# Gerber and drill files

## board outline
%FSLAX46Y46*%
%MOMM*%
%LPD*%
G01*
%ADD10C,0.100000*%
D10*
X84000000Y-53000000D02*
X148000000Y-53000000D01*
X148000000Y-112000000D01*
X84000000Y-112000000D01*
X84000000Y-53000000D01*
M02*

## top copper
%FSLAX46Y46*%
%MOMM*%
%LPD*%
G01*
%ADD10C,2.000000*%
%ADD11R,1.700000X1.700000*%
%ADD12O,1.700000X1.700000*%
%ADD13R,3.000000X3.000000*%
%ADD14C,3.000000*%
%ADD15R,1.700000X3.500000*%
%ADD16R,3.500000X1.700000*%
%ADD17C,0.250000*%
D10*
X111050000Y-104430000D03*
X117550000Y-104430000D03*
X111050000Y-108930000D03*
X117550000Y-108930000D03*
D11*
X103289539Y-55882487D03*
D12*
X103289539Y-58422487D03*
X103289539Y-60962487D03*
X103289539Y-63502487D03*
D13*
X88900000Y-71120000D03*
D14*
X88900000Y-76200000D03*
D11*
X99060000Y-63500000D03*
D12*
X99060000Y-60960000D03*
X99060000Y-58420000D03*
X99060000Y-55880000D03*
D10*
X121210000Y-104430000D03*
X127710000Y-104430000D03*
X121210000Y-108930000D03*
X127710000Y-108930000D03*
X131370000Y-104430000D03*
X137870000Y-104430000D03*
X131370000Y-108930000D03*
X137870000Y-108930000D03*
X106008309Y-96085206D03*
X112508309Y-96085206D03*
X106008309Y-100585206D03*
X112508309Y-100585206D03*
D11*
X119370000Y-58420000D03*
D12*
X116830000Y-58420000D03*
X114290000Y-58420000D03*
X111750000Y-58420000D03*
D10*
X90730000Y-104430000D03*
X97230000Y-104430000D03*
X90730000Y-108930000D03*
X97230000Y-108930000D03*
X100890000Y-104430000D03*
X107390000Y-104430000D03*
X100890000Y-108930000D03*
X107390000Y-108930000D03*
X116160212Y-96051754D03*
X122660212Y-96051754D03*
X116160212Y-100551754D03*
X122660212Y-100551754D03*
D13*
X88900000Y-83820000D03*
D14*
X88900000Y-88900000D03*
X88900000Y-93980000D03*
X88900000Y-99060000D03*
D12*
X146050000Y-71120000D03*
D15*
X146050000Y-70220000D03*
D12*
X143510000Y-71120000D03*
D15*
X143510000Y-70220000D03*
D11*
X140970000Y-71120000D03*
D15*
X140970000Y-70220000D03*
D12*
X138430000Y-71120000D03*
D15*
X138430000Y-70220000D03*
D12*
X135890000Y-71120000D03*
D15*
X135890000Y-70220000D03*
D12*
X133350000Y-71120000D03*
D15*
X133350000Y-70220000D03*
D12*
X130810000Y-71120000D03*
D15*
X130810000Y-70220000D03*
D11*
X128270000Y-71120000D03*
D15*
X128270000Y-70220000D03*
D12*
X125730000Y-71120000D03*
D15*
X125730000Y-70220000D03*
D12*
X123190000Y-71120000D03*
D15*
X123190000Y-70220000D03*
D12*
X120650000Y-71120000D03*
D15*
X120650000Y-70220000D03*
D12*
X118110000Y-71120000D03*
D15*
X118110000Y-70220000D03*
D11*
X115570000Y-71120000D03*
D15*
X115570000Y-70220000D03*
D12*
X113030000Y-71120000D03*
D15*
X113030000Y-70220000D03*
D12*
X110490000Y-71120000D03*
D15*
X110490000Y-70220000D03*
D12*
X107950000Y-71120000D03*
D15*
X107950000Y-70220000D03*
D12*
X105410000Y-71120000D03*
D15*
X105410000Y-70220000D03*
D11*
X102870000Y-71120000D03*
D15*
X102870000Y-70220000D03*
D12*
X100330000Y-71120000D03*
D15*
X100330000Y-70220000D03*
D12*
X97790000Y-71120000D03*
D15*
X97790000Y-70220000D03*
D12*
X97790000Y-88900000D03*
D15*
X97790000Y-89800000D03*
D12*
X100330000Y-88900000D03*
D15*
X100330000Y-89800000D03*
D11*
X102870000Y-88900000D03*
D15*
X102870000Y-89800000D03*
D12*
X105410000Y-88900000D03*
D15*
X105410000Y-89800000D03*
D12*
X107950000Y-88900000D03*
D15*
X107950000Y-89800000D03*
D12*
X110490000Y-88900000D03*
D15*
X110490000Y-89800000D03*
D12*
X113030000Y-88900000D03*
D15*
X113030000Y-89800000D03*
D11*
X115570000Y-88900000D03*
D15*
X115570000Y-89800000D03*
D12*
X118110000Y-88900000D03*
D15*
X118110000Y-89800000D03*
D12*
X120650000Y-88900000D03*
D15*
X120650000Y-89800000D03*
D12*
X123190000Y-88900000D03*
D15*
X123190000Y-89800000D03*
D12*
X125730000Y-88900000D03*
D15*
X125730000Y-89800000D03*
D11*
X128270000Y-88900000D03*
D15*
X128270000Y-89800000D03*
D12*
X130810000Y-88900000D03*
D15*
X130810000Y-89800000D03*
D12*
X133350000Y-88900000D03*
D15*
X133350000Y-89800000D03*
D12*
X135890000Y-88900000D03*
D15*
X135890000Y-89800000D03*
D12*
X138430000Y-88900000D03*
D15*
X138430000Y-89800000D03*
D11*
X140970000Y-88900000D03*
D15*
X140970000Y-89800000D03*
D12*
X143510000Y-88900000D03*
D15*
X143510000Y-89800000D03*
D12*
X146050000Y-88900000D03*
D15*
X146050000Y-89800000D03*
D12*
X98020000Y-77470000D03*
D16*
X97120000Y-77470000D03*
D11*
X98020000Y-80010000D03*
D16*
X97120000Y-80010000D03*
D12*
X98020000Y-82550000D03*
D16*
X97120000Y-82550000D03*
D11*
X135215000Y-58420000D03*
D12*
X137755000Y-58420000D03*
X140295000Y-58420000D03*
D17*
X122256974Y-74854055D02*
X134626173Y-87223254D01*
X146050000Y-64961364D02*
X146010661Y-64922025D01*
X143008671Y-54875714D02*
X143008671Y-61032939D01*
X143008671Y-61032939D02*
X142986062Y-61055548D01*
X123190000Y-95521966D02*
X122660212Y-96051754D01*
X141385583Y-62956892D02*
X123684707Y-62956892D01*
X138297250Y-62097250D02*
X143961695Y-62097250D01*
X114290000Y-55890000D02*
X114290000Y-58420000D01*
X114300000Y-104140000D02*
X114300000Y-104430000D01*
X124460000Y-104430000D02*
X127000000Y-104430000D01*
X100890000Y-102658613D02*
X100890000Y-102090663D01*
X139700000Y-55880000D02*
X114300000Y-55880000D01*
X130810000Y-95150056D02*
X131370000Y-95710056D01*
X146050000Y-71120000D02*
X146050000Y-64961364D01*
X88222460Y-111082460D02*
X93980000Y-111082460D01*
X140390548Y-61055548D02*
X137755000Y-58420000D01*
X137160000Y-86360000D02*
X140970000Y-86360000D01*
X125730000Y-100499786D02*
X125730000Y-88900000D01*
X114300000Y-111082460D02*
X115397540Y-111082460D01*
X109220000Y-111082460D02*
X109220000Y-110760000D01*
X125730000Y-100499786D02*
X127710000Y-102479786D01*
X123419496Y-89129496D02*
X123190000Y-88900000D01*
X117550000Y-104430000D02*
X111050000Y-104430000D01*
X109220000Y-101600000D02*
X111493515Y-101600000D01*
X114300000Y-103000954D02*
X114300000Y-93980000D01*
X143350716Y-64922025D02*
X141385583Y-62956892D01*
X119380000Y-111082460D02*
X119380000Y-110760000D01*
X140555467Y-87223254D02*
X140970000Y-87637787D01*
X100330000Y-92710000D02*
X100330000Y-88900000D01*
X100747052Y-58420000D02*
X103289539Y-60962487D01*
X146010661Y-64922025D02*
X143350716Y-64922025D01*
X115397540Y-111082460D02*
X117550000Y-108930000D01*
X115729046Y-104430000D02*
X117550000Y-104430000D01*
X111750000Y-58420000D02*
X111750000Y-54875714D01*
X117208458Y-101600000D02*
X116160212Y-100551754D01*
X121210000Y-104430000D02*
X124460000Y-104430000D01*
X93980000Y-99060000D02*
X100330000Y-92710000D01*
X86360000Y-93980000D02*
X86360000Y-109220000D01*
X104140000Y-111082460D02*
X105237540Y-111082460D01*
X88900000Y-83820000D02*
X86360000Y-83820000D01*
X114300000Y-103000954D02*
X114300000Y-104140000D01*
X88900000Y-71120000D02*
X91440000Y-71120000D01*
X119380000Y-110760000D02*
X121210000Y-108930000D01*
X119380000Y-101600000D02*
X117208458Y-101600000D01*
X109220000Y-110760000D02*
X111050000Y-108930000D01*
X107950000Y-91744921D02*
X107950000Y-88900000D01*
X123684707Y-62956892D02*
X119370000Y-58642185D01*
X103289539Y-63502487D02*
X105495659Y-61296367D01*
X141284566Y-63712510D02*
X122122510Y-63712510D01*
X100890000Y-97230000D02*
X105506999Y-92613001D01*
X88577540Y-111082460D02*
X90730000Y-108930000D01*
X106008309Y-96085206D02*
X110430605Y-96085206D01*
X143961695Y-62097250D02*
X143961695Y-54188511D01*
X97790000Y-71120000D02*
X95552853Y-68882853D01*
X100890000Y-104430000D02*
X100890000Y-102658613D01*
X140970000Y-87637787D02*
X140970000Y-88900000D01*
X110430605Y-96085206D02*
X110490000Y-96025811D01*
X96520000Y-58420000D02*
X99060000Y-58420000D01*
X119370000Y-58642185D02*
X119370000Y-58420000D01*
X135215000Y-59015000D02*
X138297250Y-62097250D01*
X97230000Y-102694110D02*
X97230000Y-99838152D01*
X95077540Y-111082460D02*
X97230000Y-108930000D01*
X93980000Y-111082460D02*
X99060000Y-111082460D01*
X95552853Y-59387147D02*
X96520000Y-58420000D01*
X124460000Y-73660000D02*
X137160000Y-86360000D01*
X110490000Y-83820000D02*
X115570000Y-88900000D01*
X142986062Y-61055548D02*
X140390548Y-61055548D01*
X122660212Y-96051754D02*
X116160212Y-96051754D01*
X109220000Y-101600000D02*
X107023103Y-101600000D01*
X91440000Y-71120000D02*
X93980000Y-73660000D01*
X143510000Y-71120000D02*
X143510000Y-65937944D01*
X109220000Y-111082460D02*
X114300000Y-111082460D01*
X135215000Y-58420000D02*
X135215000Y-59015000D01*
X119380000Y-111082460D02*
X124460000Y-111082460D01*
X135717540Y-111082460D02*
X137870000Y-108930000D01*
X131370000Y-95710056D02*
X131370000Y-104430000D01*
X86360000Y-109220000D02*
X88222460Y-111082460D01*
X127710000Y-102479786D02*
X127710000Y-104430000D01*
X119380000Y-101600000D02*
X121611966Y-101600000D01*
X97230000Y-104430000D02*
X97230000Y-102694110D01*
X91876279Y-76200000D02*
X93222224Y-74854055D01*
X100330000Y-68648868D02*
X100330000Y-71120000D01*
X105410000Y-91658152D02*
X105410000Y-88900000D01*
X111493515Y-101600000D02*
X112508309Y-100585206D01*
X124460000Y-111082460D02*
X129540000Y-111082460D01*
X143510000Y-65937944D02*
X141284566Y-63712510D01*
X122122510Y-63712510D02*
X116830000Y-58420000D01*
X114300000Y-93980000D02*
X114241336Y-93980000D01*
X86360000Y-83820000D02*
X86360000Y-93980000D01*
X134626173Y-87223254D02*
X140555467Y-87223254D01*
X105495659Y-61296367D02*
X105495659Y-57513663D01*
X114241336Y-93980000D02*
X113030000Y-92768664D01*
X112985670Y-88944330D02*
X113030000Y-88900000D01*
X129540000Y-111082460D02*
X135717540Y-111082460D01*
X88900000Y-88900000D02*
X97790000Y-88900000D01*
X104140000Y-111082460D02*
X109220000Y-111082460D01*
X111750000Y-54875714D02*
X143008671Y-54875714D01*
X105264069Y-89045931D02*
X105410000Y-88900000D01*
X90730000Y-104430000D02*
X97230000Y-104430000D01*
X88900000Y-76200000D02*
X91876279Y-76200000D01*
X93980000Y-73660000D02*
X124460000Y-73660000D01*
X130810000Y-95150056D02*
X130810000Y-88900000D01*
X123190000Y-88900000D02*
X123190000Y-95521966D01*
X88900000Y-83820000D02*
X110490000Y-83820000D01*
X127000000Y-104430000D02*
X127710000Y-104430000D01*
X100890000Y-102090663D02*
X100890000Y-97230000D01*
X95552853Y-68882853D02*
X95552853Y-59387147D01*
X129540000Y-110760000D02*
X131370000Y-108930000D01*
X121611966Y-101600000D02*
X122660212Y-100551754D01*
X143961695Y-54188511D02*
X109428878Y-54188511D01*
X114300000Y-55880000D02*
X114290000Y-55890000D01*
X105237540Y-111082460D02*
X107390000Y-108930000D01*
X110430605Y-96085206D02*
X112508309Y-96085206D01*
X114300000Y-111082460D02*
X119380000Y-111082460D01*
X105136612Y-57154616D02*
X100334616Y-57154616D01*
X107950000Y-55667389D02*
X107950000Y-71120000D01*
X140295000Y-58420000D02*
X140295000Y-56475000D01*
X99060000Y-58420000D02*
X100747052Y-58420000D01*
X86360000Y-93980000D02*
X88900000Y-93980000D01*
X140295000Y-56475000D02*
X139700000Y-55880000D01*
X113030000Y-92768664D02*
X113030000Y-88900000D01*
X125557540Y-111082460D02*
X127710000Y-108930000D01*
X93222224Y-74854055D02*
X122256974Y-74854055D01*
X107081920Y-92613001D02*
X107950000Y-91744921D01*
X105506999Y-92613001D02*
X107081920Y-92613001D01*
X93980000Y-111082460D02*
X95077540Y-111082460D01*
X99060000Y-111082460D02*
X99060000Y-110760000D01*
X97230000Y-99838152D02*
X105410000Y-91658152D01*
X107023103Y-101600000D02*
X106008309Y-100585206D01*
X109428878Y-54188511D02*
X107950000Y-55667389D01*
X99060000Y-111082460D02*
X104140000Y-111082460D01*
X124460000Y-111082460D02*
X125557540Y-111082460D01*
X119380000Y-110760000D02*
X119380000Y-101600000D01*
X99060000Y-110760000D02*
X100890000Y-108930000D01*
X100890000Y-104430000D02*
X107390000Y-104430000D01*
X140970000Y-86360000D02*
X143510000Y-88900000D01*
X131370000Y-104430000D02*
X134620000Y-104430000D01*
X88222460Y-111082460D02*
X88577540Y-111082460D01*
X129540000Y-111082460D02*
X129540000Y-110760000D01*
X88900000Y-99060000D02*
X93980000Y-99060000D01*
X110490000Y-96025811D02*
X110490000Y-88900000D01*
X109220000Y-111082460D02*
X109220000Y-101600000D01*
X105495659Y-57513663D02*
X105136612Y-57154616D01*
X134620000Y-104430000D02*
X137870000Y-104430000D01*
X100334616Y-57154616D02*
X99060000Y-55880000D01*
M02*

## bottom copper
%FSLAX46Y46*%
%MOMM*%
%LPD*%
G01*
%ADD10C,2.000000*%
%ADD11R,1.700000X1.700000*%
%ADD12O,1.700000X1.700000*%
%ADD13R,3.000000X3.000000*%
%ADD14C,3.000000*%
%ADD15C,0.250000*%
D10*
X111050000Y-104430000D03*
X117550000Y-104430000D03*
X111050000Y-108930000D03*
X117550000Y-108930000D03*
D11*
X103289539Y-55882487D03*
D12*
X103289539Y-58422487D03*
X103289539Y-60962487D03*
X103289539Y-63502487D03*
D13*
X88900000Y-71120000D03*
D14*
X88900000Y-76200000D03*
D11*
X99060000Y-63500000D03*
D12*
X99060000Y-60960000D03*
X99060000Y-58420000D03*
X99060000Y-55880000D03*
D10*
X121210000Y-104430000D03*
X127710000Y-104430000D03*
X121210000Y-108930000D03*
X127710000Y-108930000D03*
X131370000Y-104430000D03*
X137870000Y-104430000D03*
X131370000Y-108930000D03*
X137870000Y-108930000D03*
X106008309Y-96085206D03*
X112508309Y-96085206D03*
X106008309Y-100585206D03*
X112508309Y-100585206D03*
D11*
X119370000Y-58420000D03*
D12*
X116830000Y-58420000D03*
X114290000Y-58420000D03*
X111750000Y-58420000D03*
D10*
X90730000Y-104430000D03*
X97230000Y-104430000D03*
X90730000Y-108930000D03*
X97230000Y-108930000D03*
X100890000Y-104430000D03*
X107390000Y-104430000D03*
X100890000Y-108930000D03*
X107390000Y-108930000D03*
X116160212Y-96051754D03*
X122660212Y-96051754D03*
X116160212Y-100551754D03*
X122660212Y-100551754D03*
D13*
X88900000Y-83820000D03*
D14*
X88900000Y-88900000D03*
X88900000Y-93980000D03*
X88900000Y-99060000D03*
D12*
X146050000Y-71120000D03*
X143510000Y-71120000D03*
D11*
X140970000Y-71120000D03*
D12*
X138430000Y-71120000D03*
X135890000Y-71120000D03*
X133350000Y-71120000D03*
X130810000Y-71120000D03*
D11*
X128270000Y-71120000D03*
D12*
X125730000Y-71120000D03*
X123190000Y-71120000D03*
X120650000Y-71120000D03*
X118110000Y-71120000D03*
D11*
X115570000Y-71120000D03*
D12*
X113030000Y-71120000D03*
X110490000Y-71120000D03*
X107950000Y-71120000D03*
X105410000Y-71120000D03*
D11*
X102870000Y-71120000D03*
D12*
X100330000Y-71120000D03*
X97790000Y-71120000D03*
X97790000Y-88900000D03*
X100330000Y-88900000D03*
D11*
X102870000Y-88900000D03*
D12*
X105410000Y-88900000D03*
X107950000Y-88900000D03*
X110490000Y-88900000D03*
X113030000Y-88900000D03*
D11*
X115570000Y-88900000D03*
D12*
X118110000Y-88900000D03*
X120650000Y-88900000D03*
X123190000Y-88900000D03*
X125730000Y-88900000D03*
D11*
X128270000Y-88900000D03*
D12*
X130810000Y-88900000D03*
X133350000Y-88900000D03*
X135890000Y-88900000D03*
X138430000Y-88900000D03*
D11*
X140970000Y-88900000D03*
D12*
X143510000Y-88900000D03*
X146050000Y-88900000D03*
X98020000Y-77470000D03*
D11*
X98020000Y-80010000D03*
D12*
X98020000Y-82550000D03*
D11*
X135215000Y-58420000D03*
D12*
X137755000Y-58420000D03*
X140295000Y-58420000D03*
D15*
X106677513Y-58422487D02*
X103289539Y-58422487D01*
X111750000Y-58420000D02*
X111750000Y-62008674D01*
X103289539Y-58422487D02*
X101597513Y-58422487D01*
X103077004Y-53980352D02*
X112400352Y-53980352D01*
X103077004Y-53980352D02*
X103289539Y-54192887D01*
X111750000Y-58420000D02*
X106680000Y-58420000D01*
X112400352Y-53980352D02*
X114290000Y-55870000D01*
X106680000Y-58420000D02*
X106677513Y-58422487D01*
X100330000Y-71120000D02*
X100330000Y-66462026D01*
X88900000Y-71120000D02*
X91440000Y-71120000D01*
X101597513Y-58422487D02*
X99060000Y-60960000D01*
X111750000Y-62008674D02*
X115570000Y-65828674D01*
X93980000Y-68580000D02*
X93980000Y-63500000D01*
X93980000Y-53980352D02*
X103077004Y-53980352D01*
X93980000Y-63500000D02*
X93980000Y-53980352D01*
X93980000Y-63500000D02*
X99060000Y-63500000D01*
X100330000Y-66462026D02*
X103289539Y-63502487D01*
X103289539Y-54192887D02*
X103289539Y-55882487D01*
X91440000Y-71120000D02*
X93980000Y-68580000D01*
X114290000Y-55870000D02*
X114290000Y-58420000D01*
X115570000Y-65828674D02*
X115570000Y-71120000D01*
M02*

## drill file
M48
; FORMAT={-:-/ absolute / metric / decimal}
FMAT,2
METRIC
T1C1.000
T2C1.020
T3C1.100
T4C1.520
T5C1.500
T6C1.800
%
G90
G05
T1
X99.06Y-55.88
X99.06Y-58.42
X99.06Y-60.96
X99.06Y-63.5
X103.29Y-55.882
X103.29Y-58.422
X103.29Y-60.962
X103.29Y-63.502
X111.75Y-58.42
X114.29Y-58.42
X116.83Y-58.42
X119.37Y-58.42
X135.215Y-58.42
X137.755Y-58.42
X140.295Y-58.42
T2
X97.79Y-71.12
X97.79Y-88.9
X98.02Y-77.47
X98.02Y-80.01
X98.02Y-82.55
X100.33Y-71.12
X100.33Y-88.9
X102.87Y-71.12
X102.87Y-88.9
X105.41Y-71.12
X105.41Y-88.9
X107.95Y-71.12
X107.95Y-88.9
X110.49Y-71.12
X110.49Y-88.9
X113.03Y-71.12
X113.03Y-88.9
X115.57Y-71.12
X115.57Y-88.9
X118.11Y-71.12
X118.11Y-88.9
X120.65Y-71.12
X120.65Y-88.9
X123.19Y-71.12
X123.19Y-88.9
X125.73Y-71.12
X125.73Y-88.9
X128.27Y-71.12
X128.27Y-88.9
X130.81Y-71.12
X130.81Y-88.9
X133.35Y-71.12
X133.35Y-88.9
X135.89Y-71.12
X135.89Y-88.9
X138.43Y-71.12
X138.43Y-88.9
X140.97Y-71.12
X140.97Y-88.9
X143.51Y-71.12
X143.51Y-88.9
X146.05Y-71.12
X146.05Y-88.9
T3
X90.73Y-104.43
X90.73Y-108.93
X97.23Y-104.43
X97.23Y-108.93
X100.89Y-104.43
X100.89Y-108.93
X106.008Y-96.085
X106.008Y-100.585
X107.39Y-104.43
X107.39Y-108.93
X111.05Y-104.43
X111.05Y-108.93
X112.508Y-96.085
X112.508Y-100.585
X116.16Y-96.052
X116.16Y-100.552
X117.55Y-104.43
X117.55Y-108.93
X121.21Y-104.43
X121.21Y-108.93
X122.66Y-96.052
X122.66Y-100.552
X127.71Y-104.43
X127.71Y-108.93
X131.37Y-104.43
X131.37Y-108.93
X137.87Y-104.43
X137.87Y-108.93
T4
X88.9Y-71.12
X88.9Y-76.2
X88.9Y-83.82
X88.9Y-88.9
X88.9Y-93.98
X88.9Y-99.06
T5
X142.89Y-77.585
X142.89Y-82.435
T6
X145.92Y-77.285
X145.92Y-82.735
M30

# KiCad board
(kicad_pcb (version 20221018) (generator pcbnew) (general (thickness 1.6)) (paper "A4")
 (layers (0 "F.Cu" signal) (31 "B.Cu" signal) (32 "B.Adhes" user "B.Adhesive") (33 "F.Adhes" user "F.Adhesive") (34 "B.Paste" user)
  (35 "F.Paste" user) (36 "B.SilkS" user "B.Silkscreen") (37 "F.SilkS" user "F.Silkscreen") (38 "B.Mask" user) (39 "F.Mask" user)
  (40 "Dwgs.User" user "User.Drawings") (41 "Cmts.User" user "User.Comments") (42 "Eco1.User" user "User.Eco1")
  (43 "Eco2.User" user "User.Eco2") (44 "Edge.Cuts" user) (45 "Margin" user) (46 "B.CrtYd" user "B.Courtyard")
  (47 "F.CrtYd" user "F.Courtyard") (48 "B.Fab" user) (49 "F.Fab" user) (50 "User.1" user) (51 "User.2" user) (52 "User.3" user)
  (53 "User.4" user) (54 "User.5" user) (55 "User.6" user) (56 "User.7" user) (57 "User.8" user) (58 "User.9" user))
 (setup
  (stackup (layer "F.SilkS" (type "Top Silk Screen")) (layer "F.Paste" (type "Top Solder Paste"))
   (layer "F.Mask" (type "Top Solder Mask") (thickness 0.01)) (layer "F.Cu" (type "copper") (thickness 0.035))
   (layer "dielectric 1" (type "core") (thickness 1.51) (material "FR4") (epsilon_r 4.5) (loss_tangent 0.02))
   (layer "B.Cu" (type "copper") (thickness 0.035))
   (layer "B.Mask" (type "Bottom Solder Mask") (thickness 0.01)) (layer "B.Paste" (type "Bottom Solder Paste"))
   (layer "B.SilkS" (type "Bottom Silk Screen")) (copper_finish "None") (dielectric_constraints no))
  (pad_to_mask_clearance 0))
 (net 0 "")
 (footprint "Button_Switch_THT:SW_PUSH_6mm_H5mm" (layer "F.Cu") (at 111.05 104.43)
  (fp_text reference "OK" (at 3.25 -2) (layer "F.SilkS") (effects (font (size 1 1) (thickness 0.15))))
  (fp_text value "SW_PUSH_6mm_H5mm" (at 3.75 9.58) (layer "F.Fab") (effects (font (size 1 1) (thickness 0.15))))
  (pad "1" thru_hole circle (at 0 0 90) (size 2 2) (drill 1.1) (layers "*.Cu" "*.Mask"))
  (pad "1" thru_hole circle (at 6.5 0 90) (size 2 2) (drill 1.1) (layers "*.Cu" "*.Mask"))
  (pad "2" thru_hole circle (at 0 4.5 90) (size 2 2) (drill 1.1) (layers "*.Cu" "*.Mask"))
  (pad "2" thru_hole circle (at 6.5 4.5 90) (size 2 2) (drill 1.1) (layers "*.Cu" "*.Mask")))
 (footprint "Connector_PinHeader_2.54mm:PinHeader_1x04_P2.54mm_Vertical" (layer "F.Cu") (at 103.289539 55.882487)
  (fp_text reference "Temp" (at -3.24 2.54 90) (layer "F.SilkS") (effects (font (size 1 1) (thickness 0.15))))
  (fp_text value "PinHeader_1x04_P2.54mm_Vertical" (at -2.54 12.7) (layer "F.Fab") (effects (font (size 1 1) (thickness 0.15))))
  (pad "1" thru_hole rect (at 0 0) (size 1.7 1.7) (drill 1) (layers "*.Cu" "*.Mask"))
  (pad "2" thru_hole oval (at 0 2.54) (size 1.7 1.7) (drill 1) (layers "*.Cu" "*.Mask"))
  (pad "3" thru_hole oval (at 0 5.08) (size 1.7 1.7) (drill 1) (layers "*.Cu" "*.Mask"))
  (pad "4" thru_hole oval (at 0 7.62) (size 1.7 1.7) (drill 1) (layers "*.Cu" "*.Mask")))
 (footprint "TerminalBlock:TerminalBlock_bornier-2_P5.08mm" (layer "F.Cu") (at 88.9 71.12 -90)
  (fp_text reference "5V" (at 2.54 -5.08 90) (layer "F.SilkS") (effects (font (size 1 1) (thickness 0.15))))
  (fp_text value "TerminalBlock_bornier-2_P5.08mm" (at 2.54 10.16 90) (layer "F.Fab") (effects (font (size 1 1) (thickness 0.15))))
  (pad "1" thru_hole rect (at 0 0 270) (size 3 3) (drill 1.52) (layers "*.Cu" "*.Mask"))
  (pad "2" thru_hole circle (at 5.08 0 270) (size 3 3) (drill 1.52) (layers "*.Cu" "*.Mask")))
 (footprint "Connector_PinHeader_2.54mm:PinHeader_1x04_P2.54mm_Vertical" (layer "F.Cu") (at 99.06 63.5 180)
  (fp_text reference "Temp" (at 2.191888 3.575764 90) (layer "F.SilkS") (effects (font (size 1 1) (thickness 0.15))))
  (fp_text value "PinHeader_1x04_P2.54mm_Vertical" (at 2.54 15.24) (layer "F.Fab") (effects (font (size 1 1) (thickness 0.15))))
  (pad "1" thru_hole rect (at 0 0 180) (size 1.7 1.7) (drill 1) (layers "*.Cu" "*.Mask"))
  (pad "2" thru_hole oval (at 0 2.54 180) (size 1.7 1.7) (drill 1) (layers "*.Cu" "*.Mask"))
  (pad "3" thru_hole oval (at 0 5.08 180) (size 1.7 1.7) (drill 1) (layers "*.Cu" "*.Mask"))
  (pad "4" thru_hole oval (at 0 7.62 180) (size 1.7 1.7) (drill 1) (layers "*.Cu" "*.Mask")))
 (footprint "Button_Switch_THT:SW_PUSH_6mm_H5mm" (layer "F.Cu") (at 121.21 104.43)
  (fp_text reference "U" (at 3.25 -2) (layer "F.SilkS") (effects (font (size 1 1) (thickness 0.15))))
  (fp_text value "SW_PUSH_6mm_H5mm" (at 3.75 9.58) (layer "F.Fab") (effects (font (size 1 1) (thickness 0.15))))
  (pad "1" thru_hole circle (at 0 0 90) (size 2 2) (drill 1.1) (layers "*.Cu" "*.Mask"))
  (pad "1" thru_hole circle (at 6.5 0 90) (size 2 2) (drill 1.1) (layers "*.Cu" "*.Mask"))
  (pad "2" thru_hole circle (at 0 4.5 90) (size 2 2) (drill 1.1) (layers "*.Cu" "*.Mask"))
  (pad "2" thru_hole circle (at 6.5 4.5 90) (size 2 2) (drill 1.1) (layers "*.Cu" "*.Mask")))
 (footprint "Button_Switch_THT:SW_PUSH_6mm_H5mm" (layer "F.Cu") (at 131.37 104.43)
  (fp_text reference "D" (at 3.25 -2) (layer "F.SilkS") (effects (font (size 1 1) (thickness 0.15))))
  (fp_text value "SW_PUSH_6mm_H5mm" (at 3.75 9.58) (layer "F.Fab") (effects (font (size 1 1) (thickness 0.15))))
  (pad "1" thru_hole circle (at 0 0 90) (size 2 2) (drill 1.1) (layers "*.Cu" "*.Mask"))
  (pad "1" thru_hole circle (at 6.5 0 90) (size 2 2) (drill 1.1) (layers "*.Cu" "*.Mask"))
  (pad "2" thru_hole circle (at 0 4.5 90) (size 2 2) (drill 1.1) (layers "*.Cu" "*.Mask"))
  (pad "2" thru_hole circle (at 6.5 4.5 90) (size 2 2) (drill 1.1) (layers "*.Cu" "*.Mask")))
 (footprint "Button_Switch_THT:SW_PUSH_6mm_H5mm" (layer "F.Cu") (at 106.008309 96.085206)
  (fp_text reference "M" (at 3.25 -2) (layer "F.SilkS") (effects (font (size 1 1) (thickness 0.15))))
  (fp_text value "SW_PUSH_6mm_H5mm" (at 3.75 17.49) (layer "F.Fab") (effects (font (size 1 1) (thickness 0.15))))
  (pad "1" thru_hole circle (at 0 0 90) (size 2 2) (drill 1.1) (layers "*.Cu" "*.Mask"))
  (pad "1" thru_hole circle (at 6.5 0 90) (size 2 2) (drill 1.1) (layers "*.Cu" "*.Mask"))
  (pad "2" thru_hole circle (at 0 4.5 90) (size 2 2) (drill 1.1) (layers "*.Cu" "*.Mask"))
  (pad "2" thru_hole circle (at 6.5 4.5 90) (size 2 2) (drill 1.1) (layers "*.Cu" "*.Mask")))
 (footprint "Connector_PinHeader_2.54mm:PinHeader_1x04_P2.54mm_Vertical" (layer "F.Cu") (at 119.37 58.42 -90)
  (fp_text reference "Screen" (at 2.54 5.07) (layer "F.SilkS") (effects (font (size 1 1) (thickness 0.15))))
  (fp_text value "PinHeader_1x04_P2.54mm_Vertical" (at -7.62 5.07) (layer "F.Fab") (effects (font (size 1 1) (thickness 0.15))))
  (pad "1" thru_hole rect (at 0 0 270) (size 1.7 1.7) (drill 1) (layers "*.Cu" "*.Mask"))
  (pad "2" thru_hole oval (at 0 2.54 270) (size 1.7 1.7) (drill 1) (layers "*.Cu" "*.Mask"))
  (pad "3" thru_hole oval (at 0 5.08 270) (size 1.7 1.7) (drill 1) (layers "*.Cu" "*.Mask"))
  (pad "4" thru_hole oval (at 0 7.62 270) (size 1.7 1.7) (drill 1) (layers "*.Cu" "*.Mask")))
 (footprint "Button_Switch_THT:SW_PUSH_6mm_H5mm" (layer "F.Cu") (at 90.73 104.43)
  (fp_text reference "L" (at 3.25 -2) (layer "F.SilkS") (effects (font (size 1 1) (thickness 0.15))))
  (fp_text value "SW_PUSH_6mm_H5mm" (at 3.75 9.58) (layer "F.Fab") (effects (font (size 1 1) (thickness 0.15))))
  (pad "1" thru_hole circle (at 0 0 90) (size 2 2) (drill 1.1) (layers "*.Cu" "*.Mask"))
  (pad "1" thru_hole circle (at 6.5 0 90) (size 2 2) (drill 1.1) (layers "*.Cu" "*.Mask"))
  (pad "2" thru_hole circle (at 0 4.5 90) (size 2 2) (drill 1.1) (layers "*.Cu" "*.Mask"))
  (pad "2" thru_hole circle (at 6.5 4.5 90) (size 2 2) (drill 1.1) (layers "*.Cu" "*.Mask")))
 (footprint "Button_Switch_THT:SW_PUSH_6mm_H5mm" (layer "F.Cu") (at 100.89 104.43)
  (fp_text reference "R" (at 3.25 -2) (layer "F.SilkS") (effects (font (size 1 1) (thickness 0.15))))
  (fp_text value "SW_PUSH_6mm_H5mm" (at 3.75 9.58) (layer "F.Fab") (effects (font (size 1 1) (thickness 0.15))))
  (pad "1" thru_hole circle (at 0 0 90) (size 2 2) (drill 1.1) (layers "*.Cu" "*.Mask"))
  (pad "1" thru_hole circle (at 6.5 0 90) (size 2 2) (drill 1.1) (layers "*.Cu" "*.Mask"))
  (pad "2" thru_hole circle (at 0 4.5 90) (size 2 2) (drill 1.1) (layers "*.Cu" "*.Mask"))
  (pad "2" thru_hole circle (at 6.5 4.5 90) (size 2 2) (drill 1.1) (layers "*.Cu" "*.Mask")))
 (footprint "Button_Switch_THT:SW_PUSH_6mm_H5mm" (layer "F.Cu") (at 116.160212 96.051754)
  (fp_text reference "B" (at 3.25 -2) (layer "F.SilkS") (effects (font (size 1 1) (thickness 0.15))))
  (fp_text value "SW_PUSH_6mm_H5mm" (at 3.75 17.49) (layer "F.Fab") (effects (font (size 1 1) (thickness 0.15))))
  (pad "1" thru_hole circle (at 0 0 90) (size 2 2) (drill 1.1) (layers "*.Cu" "*.Mask"))
  (pad "1" thru_hole circle (at 6.5 0 90) (size 2 2) (drill 1.1) (layers "*.Cu" "*.Mask"))
  (pad "2" thru_hole circle (at 0 4.5 90) (size 2 2) (drill 1.1) (layers "*.Cu" "*.Mask"))
  (pad "2" thru_hole circle (at 6.5 4.5 90) (size 2 2) (drill 1.1) (layers "*.Cu" "*.Mask")))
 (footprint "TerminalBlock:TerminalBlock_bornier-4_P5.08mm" (layer "F.Cu") (at 88.9 83.82 -90)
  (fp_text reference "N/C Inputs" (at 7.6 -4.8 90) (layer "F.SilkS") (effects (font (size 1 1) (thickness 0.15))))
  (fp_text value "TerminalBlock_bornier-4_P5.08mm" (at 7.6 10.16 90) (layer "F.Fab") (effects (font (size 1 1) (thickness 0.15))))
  (pad "1" thru_hole rect (at 0 0 270) (size 3 3) (drill 1.52) (layers "*.Cu" "*.Mask"))
  (pad "2" thru_hole circle (at 5.08 0 270) (size 3 3) (drill 1.52) (layers "*.Cu" "*.Mask"))
  (pad "3" thru_hole circle (at 10.16 0 270) (size 3 3) (drill 1.52) (layers "*.Cu" "*.Mask"))
  (pad "4" thru_hole circle (at 15.24 0 270) (size 3 3) (drill 1.52) (layers "*.Cu" "*.Mask")))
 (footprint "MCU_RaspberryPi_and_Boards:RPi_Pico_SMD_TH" (layer "F.Cu") (at 121.92 80.01 -90)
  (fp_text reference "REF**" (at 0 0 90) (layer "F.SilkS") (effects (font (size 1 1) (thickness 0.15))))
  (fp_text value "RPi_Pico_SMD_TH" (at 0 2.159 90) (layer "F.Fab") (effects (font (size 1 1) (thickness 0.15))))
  (pad "" np_thru_hole oval (at -2.725 -24 270) (size 1.8 1.8) (drill 1.8) (layers "*.Cu" "*.Mask"))
  (pad "" np_thru_hole oval (at -2.425 -20.97 270) (size 1.5 1.5) (drill 1.5) (layers "*.Cu" "*.Mask"))
  (pad "" np_thru_hole oval (at 2.425 -20.97 270) (size 1.5 1.5) (drill 1.5) (layers "*.Cu" "*.Mask"))
  (pad "" np_thru_hole oval (at 2.725 -24 270) (size 1.8 1.8) (drill 1.8) (layers "*.Cu" "*.Mask"))
  (pad "1" thru_hole oval (at -8.89 -24.13 270) (size 1.7 1.7) (drill 1.02) (layers "*.Cu" "*.Mask"))
  (pad "1" smd rect (at -8.89 -24.13 270) (size 3.5 1.7) (drill (offset -0.9 0)) (layers "F.Cu" "F.Mask"))
  (pad "2" thru_hole oval (at -8.89 -21.59 270) (size 1.7 1.7) (drill 1.02) (layers "*.Cu" "*.Mask"))
  (pad "2" smd rect (at -8.89 -21.59 270) (size 3.5 1.7) (drill (offset -0.9 0)) (layers "F.Cu" "F.Mask"))
  (pad "3" thru_hole rect (at -8.89 -19.05 270) (size 1.7 1.7) (drill 1.02) (layers "*.Cu" "*.Mask"))
  (pad "3" smd rect (at -8.89 -19.05 270) (size 3.5 1.7) (drill (offset -0.9 0)) (layers "F.Cu" "F.Mask"))
  (pad "4" thru_hole oval (at -8.89 -16.51 270) (size 1.7 1.7) (drill 1.02) (layers "*.Cu" "*.Mask"))
  (pad "4" smd rect (at -8.89 -16.51 270) (size 3.5 1.7) (drill (offset -0.9 0)) (layers "F.Cu" "F.Mask"))
  (pad "5" thru_hole oval (at -8.89 -13.97 270) (size 1.7 1.7) (drill 1.02) (layers "*.Cu" "*.Mask"))
  (pad "5" smd rect (at -8.89 -13.97 270) (size 3.5 1.7) (drill (offset -0.9 0)) (layers "F.Cu" "F.Mask"))
  (pad "6" thru_hole oval (at -8.89 -11.43 270) (size 1.7 1.7) (drill 1.02) (layers "*.Cu" "*.Mask"))
  (pad "6" smd rect (at -8.89 -11.43 270) (size 3.5 1.7) (drill (offset -0.9 0)) (layers "F.Cu" "F.Mask"))
  (pad "7" thru_hole oval (at -8.89 -8.89 270) (size 1.7 1.7) (drill 1.02) (layers "*.Cu" "*.Mask"))
  (pad "7" smd rect (at -8.89 -8.89 270) (size 3.5 1.7) (drill (offset -0.9 0)) (layers "F.Cu" "F.Mask"))
  (pad "8" thru_hole rect (at -8.89 -6.35 270) (size 1.7 1.7) (drill 1.02) (layers "*.Cu" "*.Mask"))
  (pad "8" smd rect (at -8.89 -6.35 270) (size 3.5 1.7) (drill (offset -0.9 0)) (layers "F.Cu" "F.Mask"))
  (pad "9" thru_hole oval (at -8.89 -3.81 270) (size 1.7 1.7) (drill 1.02) (layers "*.Cu" "*.Mask"))
  (pad "9" smd rect (at -8.89 -3.81 270) (size 3.5 1.7) (drill (offset -0.9 0)) (layers "F.Cu" "F.Mask"))
  (pad "10" thru_hole oval (at -8.89 -1.27 270) (size 1.7 1.7) (drill 1.02) (layers "*.Cu" "*.Mask"))
  (pad "10" smd rect (at -8.89 -1.27 270) (size 3.5 1.7) (drill (offset -0.9 0)) (layers "F.Cu" "F.Mask"))
  (pad "11" thru_hole oval (at -8.89 1.27 270) (size 1.7 1.7) (drill 1.02) (layers "*.Cu" "*.Mask"))
  (pad "11" smd rect (at -8.89 1.27 270) (size 3.5 1.7) (drill (offset -0.9 0)) (layers "F.Cu" "F.Mask"))
  (pad "12" thru_hole oval (at -8.89 3.81 270) (size 1.7 1.7) (drill 1.02) (layers "*.Cu" "*.Mask"))
  (pad "12" smd rect (at -8.89 3.81 270) (size 3.5 1.7) (drill (offset -0.9 0)) (layers "F.Cu" "F.Mask"))
  (pad "13" thru_hole rect (at -8.89 6.35 270) (size 1.7 1.7) (drill 1.02) (layers "*.Cu" "*.Mask"))
  (pad "13" smd rect (at -8.89 6.35 270) (size 3.5 1.7) (drill (offset -0.9 0)) (layers "F.Cu" "F.Mask"))
  (pad "14" thru_hole oval (at -8.89 8.89 270) (size 1.7 1.7) (drill 1.02) (layers "*.Cu" "*.Mask"))
  (pad "14" smd rect (at -8.89 8.89 270) (size 3.5 1.7) (drill (offset -0.9 0)) (layers "F.Cu" "F.Mask"))
  (pad "15" thru_hole oval (at -8.89 11.43 270) (size 1.7 1.7) (drill 1.02) (layers "*.Cu" "*.Mask"))
  (pad "15" smd rect (at -8.89 11.43 270) (size 3.5 1.7) (drill (offset -0.9 0)) (layers "F.Cu" "F.Mask"))
  (pad "16" thru_hole oval (at -8.89 13.97 270) (size 1.7 1.7) (drill 1.02) (layers "*.Cu" "*.Mask"))
  (pad "16" smd rect (at -8.89 13.97 270) (size 3.5 1.7) (drill (offset -0.9 0)) (layers "F.Cu" "F.Mask"))
  (pad "17" thru_hole oval (at -8.89 16.51 270) (size 1.7 1.7) (drill 1.02) (layers "*.Cu" "*.Mask"))
  (pad "17" smd rect (at -8.89 16.51 270) (size 3.5 1.7) (drill (offset -0.9 0)) (layers "F.Cu" "F.Mask"))
  (pad "18" thru_hole rect (at -8.89 19.05 270) (size 1.7 1.7) (drill 1.02) (layers "*.Cu" "*.Mask"))
  (pad "18" smd rect (at -8.89 19.05 270) (size 3.5 1.7) (drill (offset -0.9 0)) (layers "F.Cu" "F.Mask"))
  (pad "19" thru_hole oval (at -8.89 21.59 270) (size 1.7 1.7) (drill 1.02) (layers "*.Cu" "*.Mask"))
  (pad "19" smd rect (at -8.89 21.59 270) (size 3.5 1.7) (drill (offset -0.9 0)) (layers "F.Cu" "F.Mask"))
  (pad "20" thru_hole oval (at -8.89 24.13 270) (size 1.7 1.7) (drill 1.02) (layers "*.Cu" "*.Mask"))
  (pad "20" smd rect (at -8.89 24.13 270) (size 3.5 1.7) (drill (offset -0.9 0)) (layers "F.Cu" "F.Mask"))
  (pad "21" thru_hole oval (at 8.89 24.13 270) (size 1.7 1.7) (drill 1.02) (layers "*.Cu" "*.Mask"))
  (pad "21" smd rect (at 8.89 24.13 270) (size 3.5 1.7) (drill (offset 0.9 0)) (layers "F.Cu" "F.Mask"))
  (pad "22" thru_hole oval (at 8.89 21.59 270) (size 1.7 1.7) (drill 1.02) (layers "*.Cu" "*.Mask"))
  (pad "22" smd rect (at 8.89 21.59 270) (size 3.5 1.7) (drill (offset 0.9 0)) (layers "F.Cu" "F.Mask"))
  (pad "23" thru_hole rect (at 8.89 19.05 270) (size 1.7 1.7) (drill 1.02) (layers "*.Cu" "*.Mask"))
  (pad "23" smd rect (at 8.89 19.05 270) (size 3.5 1.7) (drill (offset 0.9 0)) (layers "F.Cu" "F.Mask"))
  (pad "24" thru_hole oval (at 8.89 16.51 270) (size 1.7 1.7) (drill 1.02) (layers "*.Cu" "*.Mask"))
  (pad "24" smd rect (at 8.89 16.51 270) (size 3.5 1.7) (drill (offset 0.9 0)) (layers "F.Cu" "F.Mask"))
  (pad "25" thru_hole oval (at 8.89 13.97 270) (size 1.7 1.7) (drill 1.02) (layers "*.Cu" "*.Mask"))
  (pad "25" smd rect (at 8.89 13.97 270) (size 3.5 1.7) (drill (offset 0.9 0)) (layers "F.Cu" "F.Mask"))
  (pad "26" thru_hole oval (at 8.89 11.43 270) (size 1.7 1.7) (drill 1.02) (layers "*.Cu" "*.Mask"))
  (pad "26" smd rect (at 8.89 11.43 270) (size 3.5 1.7) (drill (offset 0.9 0)) (layers "F.Cu" "F.Mask"))
  (pad "27" thru_hole oval (at 8.89 8.89 270) (size 1.7 1.7) (drill 1.02) (layers "*.Cu" "*.Mask"))
  (pad "27" smd rect (at 8.89 8.89 270) (size 3.5 1.7) (drill (offset 0.9 0)) (layers "F.Cu" "F.Mask"))
  (pad "28" thru_hole rect (at 8.89 6.35 270) (size 1.7 1.7) (drill 1.02) (layers "*.Cu" "*.Mask"))
  (pad "28" smd rect (at 8.89 6.35 270) (size 3.5 1.7) (drill (offset 0.9 0)) (layers "F.Cu" "F.Mask"))
  (pad "29" thru_hole oval (at 8.89 3.81 270) (size 1.7 1.7) (drill 1.02) (layers "*.Cu" "*.Mask"))
  (pad "29" smd rect (at 8.89 3.81 270) (size 3.5 1.7) (drill (offset 0.9 0)) (layers "F.Cu" "F.Mask"))
  (pad "30" thru_hole oval (at 8.89 1.27 270) (size 1.7 1.7) (drill 1.02) (layers "*.Cu" "*.Mask"))
  (pad "30" smd rect (at 8.89 1.27 270) (size 3.5 1.7) (drill (offset 0.9 0)) (layers "F.Cu" "F.Mask"))
  (pad "31" thru_hole oval (at 8.89 -1.27 270) (size 1.7 1.7) (drill 1.02) (layers "*.Cu" "*.Mask"))
  (pad "31" smd rect (at 8.89 -1.27 270) (size 3.5 1.7) (drill (offset 0.9 0)) (layers "F.Cu" "F.Mask"))
  (pad "32" thru_hole oval (at 8.89 -3.81 270) (size 1.7 1.7) (drill 1.02) (layers "*.Cu" "*.Mask"))
  (pad "32" smd rect (at 8.89 -3.81 270) (size 3.5 1.7) (drill (offset 0.9 0)) (layers "F.Cu" "F.Mask"))
  (pad "33" thru_hole rect (at 8.89 -6.35 270) (size 1.7 1.7) (drill 1.02) (layers "*.Cu" "*.Mask"))
  (pad "33" smd rect (at 8.89 -6.35 270) (size 3.5 1.7) (drill (offset 0.9 0)) (layers "F.Cu" "F.Mask"))
  (pad "34" thru_hole oval (at 8.89 -8.89 270) (size 1.7 1.7) (drill 1.02) (layers "*.Cu" "*.Mask"))
  (pad "34" smd rect (at 8.89 -8.89 270) (size 3.5 1.7) (drill (offset 0.9 0)) (layers "F.Cu" "F.Mask"))
  (pad "35" thru_hole oval (at 8.89 -11.43 270) (size 1.7 1.7) (drill 1.02) (layers "*.Cu" "*.Mask"))
  (pad "35" smd rect (at 8.89 -11.43 270) (size 3.5 1.7) (drill (offset 0.9 0)) (layers "F.Cu" "F.Mask"))
  (pad "36" thru_hole oval (at 8.89 -13.97 270) (size 1.7 1.7) (drill 1.02) (layers "*.Cu" "*.Mask"))
  (pad "36" smd rect (at 8.89 -13.97 270) (size 3.5 1.7) (drill (offset 0.9 0)) (layers "F.Cu" "F.Mask"))
  (pad "37" thru_hole oval (at 8.89 -16.51 270) (size 1.7 1.7) (drill 1.02) (layers "*.Cu" "*.Mask"))
  (pad "37" smd rect (at 8.89 -16.51 270) (size 3.5 1.7) (drill (offset 0.9 0)) (layers "F.Cu" "F.Mask"))
  (pad "38" thru_hole rect (at 8.89 -19.05 270) (size 1.7 1.7) (drill 1.02) (layers "*.Cu" "*.Mask"))
  (pad "38" smd rect (at 8.89 -19.05 270) (size 3.5 1.7) (drill (offset 0.9 0)) (layers "F.Cu" "F.Mask"))
  (pad "39" thru_hole oval (at 8.89 -21.59 270) (size 1.7 1.7) (drill 1.02) (layers "*.Cu" "*.Mask"))
  (pad "39" smd rect (at 8.89 -21.59 270) (size 3.5 1.7) (drill (offset 0.9 0)) (layers "F.Cu" "F.Mask"))
  (pad "40" thru_hole oval (at 8.89 -24.13 270) (size 1.7 1.7) (drill 1.02) (layers "*.Cu" "*.Mask"))
  (pad "40" smd rect (at 8.89 -24.13 270) (size 3.5 1.7) (drill (offset 0.9 0)) (layers "F.Cu" "F.Mask"))
  (pad "41" thru_hole oval (at -2.54 23.9 270) (size 1.7 1.7) (drill 1.02) (layers "*.Cu" "*.Mask"))
  (pad "41" smd rect (at -2.54 23.9) (size 3.5 1.7) (drill (offset -0.9 0)) (layers "F.Cu" "F.Mask"))
  (pad "42" thru_hole rect (at 0 23.9 270) (size 1.7 1.7) (drill 1.02) (layers "*.Cu" "*.Mask"))
  (pad "42" smd rect (at 0 23.9) (size 3.5 1.7) (drill (offset -0.9 0)) (layers "F.Cu" "F.Mask"))
  (pad "43" thru_hole oval (at 2.54 23.9 270) (size 1.7 1.7) (drill 1.02) (layers "*.Cu" "*.Mask"))
  (pad "43" smd rect (at 2.54 23.9) (size 3.5 1.7) (drill (offset -0.9 0)) (layers "F.Cu" "F.Mask")))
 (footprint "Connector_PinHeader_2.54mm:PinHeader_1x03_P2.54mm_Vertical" (layer "F.Cu") (at 135.215 58.42 90)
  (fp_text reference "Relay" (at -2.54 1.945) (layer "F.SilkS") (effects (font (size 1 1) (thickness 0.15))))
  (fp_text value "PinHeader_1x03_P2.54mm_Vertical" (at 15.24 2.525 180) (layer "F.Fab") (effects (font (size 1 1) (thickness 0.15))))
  (pad "1" thru_hole rect (at 0 0 90) (size 1.7 1.7) (drill 1) (layers "*.Cu" "*.Mask"))
  (pad "2" thru_hole oval (at 0 2.54 90) (size 1.7 1.7) (drill 1) (layers "*.Cu" "*.Mask"))
  (pad "3" thru_hole oval (at 0 5.08 90) (size 1.7 1.7) (drill 1) (layers "*.Cu" "*.Mask")))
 (gr_rect (start 84 53) (end 148 112) (stroke (width 0.1) (type default)) (fill none) (layer "Edge.Cuts"))
 (segment (start 122.256974 74.854055) (end 134.626173 87.223254) (width 0.25) (layer "F.Cu") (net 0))
 (segment (start 146.05 64.961364) (end 146.010661 64.922025) (width 0.25) (layer "F.Cu") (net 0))
 (segment (start 143.008671 54.875714) (end 143.008671 61.032939) (width 0.25) (layer "F.Cu") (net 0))
 (segment (start 143.008671 61.032939) (end 142.986062 61.055548) (width 0.25) (layer "F.Cu") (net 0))
 (segment (start 123.19 95.521966) (end 122.660212 96.051754) (width 0.25) (layer "F.Cu") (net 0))
 (segment (start 141.385583 62.956892) (end 123.684707 62.956892) (width 0.25) (layer "F.Cu") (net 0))
 (segment (start 138.29725 62.09725) (end 143.961695 62.09725) (width 0.25) (layer "F.Cu") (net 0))
 (segment (start 114.29 55.89) (end 114.29 58.42) (width 0.25) (layer "F.Cu") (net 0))
 (segment (start 114.3 104.14) (end 114.3 104.43) (width 0.25) (layer "F.Cu") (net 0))
 (segment (start 124.46 104.43) (end 127 104.43) (width 0.25) (layer "F.Cu") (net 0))
 (segment (start 100.89 102.658613) (end 100.89 102.090663) (width 0.25) (layer "F.Cu") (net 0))
 (segment (start 139.7 55.88) (end 114.3 55.88) (width 0.25) (layer "F.Cu") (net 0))
 (segment (start 130.81 95.150056) (end 131.37 95.710056) (width 0.25) (layer "F.Cu") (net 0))
 (segment (start 146.05 71.12) (end 146.05 64.961364) (width 0.25) (layer "F.Cu") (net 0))
 (segment (start 88.22246 111.08246) (end 93.98 111.08246) (width 0.25) (layer "F.Cu") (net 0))
 (segment (start 140.390548 61.055548) (end 137.755 58.42) (width 0.25) (layer "F.Cu") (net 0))
 (segment (start 137.16 86.36) (end 140.97 86.36) (width 0.25) (layer "F.Cu") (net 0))
 (segment (start 125.73 100.499786) (end 125.73 88.9) (width 0.25) (layer "F.Cu") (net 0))
 (segment (start 114.3 111.08246) (end 115.39754 111.08246) (width 0.25) (layer "F.Cu") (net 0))
 (segment (start 109.22 111.08246) (end 109.22 110.76) (width 0.25) (layer "F.Cu") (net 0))
 (segment (start 125.73 100.499786) (end 127.71 102.479786) (width 0.25) (layer "F.Cu") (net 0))
 (segment (start 123.419496 89.129496) (end 123.19 88.9) (width 0.25) (layer "F.Cu") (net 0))
 (segment (start 117.55 104.43) (end 111.05 104.43) (width 0.25) (layer "F.Cu") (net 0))
 (segment (start 109.22 101.6) (end 111.493515 101.6) (width 0.25) (layer "F.Cu") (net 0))
 (segment (start 114.3 103.000954) (end 114.3 93.98) (width 0.25) (layer "F.Cu") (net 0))
 (segment (start 143.350716 64.922025) (end 141.385583 62.956892) (width 0.25) (layer "F.Cu") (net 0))
 (segment (start 119.38 111.08246) (end 119.38 110.76) (width 0.25) (layer "F.Cu") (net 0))
 (segment (start 140.555467 87.223254) (end 140.97 87.637787) (width 0.25) (layer "F.Cu") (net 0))
 (segment (start 100.33 92.71) (end 100.33 88.9) (width 0.25) (layer "F.Cu") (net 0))
 (segment (start 100.747052 58.42) (end 103.289539 60.962487) (width 0.25) (layer "F.Cu") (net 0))
 (segment (start 146.010661 64.922025) (end 143.350716 64.922025) (width 0.25) (layer "F.Cu") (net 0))
 (segment (start 115.39754 111.08246) (end 117.55 108.93) (width 0.25) (layer "F.Cu") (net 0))
 (segment (start 115.729046 104.43) (end 117.55 104.43) (width 0.25) (layer "F.Cu") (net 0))
 (segment (start 111.75 58.42) (end 111.75 54.875714) (width 0.25) (layer "F.Cu") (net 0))
 (segment (start 117.208458 101.6) (end 116.160212 100.551754) (width 0.25) (layer "F.Cu") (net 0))
 (segment (start 121.21 104.43) (end 124.46 104.43) (width 0.25) (layer "F.Cu") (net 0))
 (segment (start 93.98 99.06) (end 100.33 92.71) (width 0.25) (layer "F.Cu") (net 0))
 (segment (start 86.36 93.98) (end 86.36 109.22) (width 0.25) (layer "F.Cu") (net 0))
 (segment (start 104.14 111.08246) (end 105.23754 111.08246) (width 0.25) (layer "F.Cu") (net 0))
 (segment (start 88.9 83.82) (end 86.36 83.82) (width 0.25) (layer "F.Cu") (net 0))
 (segment (start 114.3 103.000954) (end 114.3 104.14) (width 0.25) (layer "F.Cu") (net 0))
 (segment (start 88.9 71.12) (end 91.44 71.12) (width 0.25) (layer "F.Cu") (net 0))
 (segment (start 119.38 110.76) (end 121.21 108.93) (width 0.25) (layer "F.Cu") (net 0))
 (segment (start 119.38 101.6) (end 117.208458 101.6) (width 0.25) (layer "F.Cu") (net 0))
 (segment (start 109.22 110.76) (end 111.05 108.93) (width 0.25) (layer "F.Cu") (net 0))
 (segment (start 107.95 91.744921) (end 107.95 88.9) (width 0.25) (layer "F.Cu") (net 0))
 (segment (start 123.684707 62.956892) (end 119.37 58.642185) (width 0.25) (layer "F.Cu") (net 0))
 (segment (start 103.289539 63.502487) (end 105.495659 61.296367) (width 0.25) (layer "F.Cu") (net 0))
 (segment (start 141.284566 63.71251) (end 122.12251 63.71251) (width 0.25) (layer "F.Cu") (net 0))
 (segment (start 100.89 97.23) (end 105.506999 92.613001) (width 0.25) (layer "F.Cu") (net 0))
 (segment (start 88.57754 111.08246) (end 90.73 108.93) (width 0.25) (layer "F.Cu") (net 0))
 (segment (start 106.008309 96.085206) (end 110.430605 96.085206) (width 0.25) (layer "F.Cu") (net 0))
 (segment (start 143.961695 62.09725) (end 143.961695 54.188511) (width 0.25) (layer "F.Cu") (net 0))
 (segment (start 97.79 71.12) (end 95.552853 68.882853) (width 0.25) (layer "F.Cu") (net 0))
 (segment (start 100.89 104.43) (end 100.89 102.658613) (width 0.25) (layer "F.Cu") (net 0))
 (segment (start 140.97 87.637787) (end 140.97 88.9) (width 0.25) (layer "F.Cu") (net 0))
 (segment (start 110.430605 96.085206) (end 110.49 96.025811) (width 0.25) (layer "F.Cu") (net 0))
 (segment (start 96.52 58.42) (end 99.06 58.42) (width 0.25) (layer "F.Cu") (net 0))
 (segment (start 119.37 58.642185) (end 119.37 58.42) (width 0.25) (layer "F.Cu") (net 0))
 (segment (start 135.215 59.015) (end 138.29725 62.09725) (width 0.25) (layer "F.Cu") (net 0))
 (segment (start 97.23 102.69411) (end 97.23 99.838152) (width 0.25) (layer "F.Cu") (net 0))
 (segment (start 95.07754 111.08246) (end 97.23 108.93) (width 0.25) (layer "F.Cu") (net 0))
 (segment (start 93.98 111.08246) (end 99.06 111.08246) (width 0.25) (layer "F.Cu") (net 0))
 (segment (start 95.552853 59.387147) (end 96.52 58.42) (width 0.25) (layer "F.Cu") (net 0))
 (segment (start 124.46 73.66) (end 137.16 86.36) (width 0.25) (layer "F.Cu") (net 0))
 (segment (start 110.49 83.82) (end 115.57 88.9) (width 0.25) (layer "F.Cu") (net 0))
 (segment (start 142.986062 61.055548) (end 140.390548 61.055548) (width 0.25) (layer "F.Cu") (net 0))
 (segment (start 122.660212 96.051754) (end 116.160212 96.051754) (width 0.25) (layer "F.Cu") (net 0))
 (segment (start 109.22 101.6) (end 107.023103 101.6) (width 0.25) (layer "F.Cu") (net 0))
 (segment (start 91.44 71.12) (end 93.98 73.66) (width 0.25) (layer "F.Cu") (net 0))
 (segment (start 143.51 71.12) (end 143.51 65.937944) (width 0.25) (layer "F.Cu") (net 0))
 (segment (start 109.22 111.08246) (end 114.3 111.08246) (width 0.25) (layer "F.Cu") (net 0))
 (segment (start 135.215 58.42) (end 135.215 59.015) (width 0.25) (layer "F.Cu") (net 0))
 (segment (start 119.38 111.08246) (end 124.46 111.08246) (width 0.25) (layer "F.Cu") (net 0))
 (segment (start 135.71754 111.08246) (end 137.87 108.93) (width 0.25) (layer "F.Cu") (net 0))
 (segment (start 131.37 95.710056) (end 131.37 104.43) (width 0.25) (layer "F.Cu") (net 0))
 (segment (start 86.36 109.22) (end 88.22246 111.08246) (width 0.25) (layer "F.Cu") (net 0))
 (segment (start 127.71 102.479786) (end 127.71 104.43) (width 0.25) (layer "F.Cu") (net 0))
 (segment (start 119.38 101.6) (end 121.611966 101.6) (width 0.25) (layer "F.Cu") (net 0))
 (segment (start 97.23 104.43) (end 97.23 102.69411) (width 0.25) (layer "F.Cu") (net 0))
 (segment (start 91.876279 76.2) (end 93.222224 74.854055) (width 0.25) (layer "F.Cu") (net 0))
 (segment (start 100.33 68.648868) (end 100.33 71.12) (width 0.25) (layer "F.Cu") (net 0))
 (segment (start 105.41 91.658152) (end 105.41 88.9) (width 0.25) (layer "F.Cu") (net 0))
 (segment (start 111.493515 101.6) (end 112.508309 100.585206) (width 0.25) (layer "F.Cu") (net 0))
 (segment (start 124.46 111.08246) (end 129.54 111.08246) (width 0.25) (layer "F.Cu") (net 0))
 (segment (start 143.51 65.937944) (end 141.284566 63.71251) (width 0.25) (layer "F.Cu") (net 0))
 (segment (start 122.12251 63.71251) (end 116.83 58.42) (width 0.25) (layer "F.Cu") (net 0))
 (segment (start 114.3 93.98) (end 114.241336 93.98) (width 0.25) (layer "F.Cu") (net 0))
 (segment (start 86.36 83.82) (end 86.36 93.98) (width 0.25) (layer "F.Cu") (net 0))
 (segment (start 134.626173 87.223254) (end 140.555467 87.223254) (width 0.25) (layer "F.Cu") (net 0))
 (segment (start 105.495659 61.296367) (end 105.495659 57.513663) (width 0.25) (layer "F.Cu") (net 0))
 (segment (start 114.241336 93.98) (end 113.03 92.768664) (width 0.25) (layer "F.Cu") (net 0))
 (segment (start 112.98567 88.94433) (end 113.03 88.9) (width 0.25) (layer "F.Cu") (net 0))
 (segment (start 129.54 111.08246) (end 135.71754 111.08246) (width 0.25) (layer "F.Cu") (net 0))
 (segment (start 88.9 88.9) (end 97.79 88.9) (width 0.25) (layer "F.Cu") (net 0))
 (segment (start 104.14 111.08246) (end 109.22 111.08246) (width 0.25) (layer "F.Cu") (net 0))
 (segment (start 111.75 54.875714) (end 143.008671 54.875714) (width 0.25) (layer "F.Cu") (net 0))
 (segment (start 105.264069 89.045931) (end 105.41 88.9) (width 0.25) (layer "F.Cu") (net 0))
 (segment (start 90.73 104.43) (end 97.23 104.43) (width 0.25) (layer "F.Cu") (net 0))
 (segment (start 88.9 76.2) (end 91.876279 76.2) (width 0.25) (layer "F.Cu") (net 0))
 (segment (start 93.98 73.66) (end 124.46 73.66) (width 0.25) (layer "F.Cu") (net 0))
 (segment (start 130.81 95.150056) (end 130.81 88.9) (width 0.25) (layer "F.Cu") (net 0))
 (segment (start 123.19 88.9) (end 123.19 95.521966) (width 0.25) (layer "F.Cu") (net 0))
 (segment (start 88.9 83.82) (end 110.49 83.82) (width 0.25) (layer "F.Cu") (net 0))
 (segment (start 127 104.43) (end 127.71 104.43) (width 0.25) (layer "F.Cu") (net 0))
 (segment (start 100.89 102.090663) (end 100.89 97.23) (width 0.25) (layer "F.Cu") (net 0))
 (segment (start 95.552853 68.882853) (end 95.552853 59.387147) (width 0.25) (layer "F.Cu") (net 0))
 (segment (start 129.54 110.76) (end 131.37 108.93) (width 0.25) (layer "F.Cu") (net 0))
 (segment (start 121.611966 101.6) (end 122.660212 100.551754) (width 0.25) (layer "F.Cu") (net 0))
 (segment (start 143.961695 54.188511) (end 109.428878 54.188511) (width 0.25) (layer "F.Cu") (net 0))
 (segment (start 114.3 55.88) (end 114.29 55.89) (width 0.25) (layer "F.Cu") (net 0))
 (segment (start 105.23754 111.08246) (end 107.39 108.93) (width 0.25) (layer "F.Cu") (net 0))
 (segment (start 110.430605 96.085206) (end 112.508309 96.085206) (width 0.25) (layer "F.Cu") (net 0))
 (segment (start 114.3 111.08246) (end 119.38 111.08246) (width 0.25) (layer "F.Cu") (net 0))
 (segment (start 105.136612 57.154616) (end 100.334616 57.154616) (width 0.25) (layer "F.Cu") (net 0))
 (segment (start 107.95 55.667389) (end 107.95 71.12) (width 0.25) (layer "F.Cu") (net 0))
 (segment (start 140.295 58.42) (end 140.295 56.475) (width 0.25) (layer "F.Cu") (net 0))
 (segment (start 99.06 58.42) (end 100.747052 58.42) (width 0.25) (layer "F.Cu") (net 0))
 (segment (start 86.36 93.98) (end 88.9 93.98) (width 0.25) (layer "F.Cu") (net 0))
 (segment (start 140.295 56.475) (end 139.7 55.88) (width 0.25) (layer "F.Cu") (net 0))
 (segment (start 113.03 92.768664) (end 113.03 88.9) (width 0.25) (layer "F.Cu") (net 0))
 (segment (start 125.55754 111.08246) (end 127.71 108.93) (width 0.25) (layer "F.Cu") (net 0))
 (segment (start 93.222224 74.854055) (end 122.256974 74.854055) (width 0.25) (layer "F.Cu") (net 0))
 (segment (start 107.08192 92.613001) (end 107.95 91.744921) (width 0.25) (layer "F.Cu") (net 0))
 (segment (start 105.506999 92.613001) (end 107.08192 92.613001) (width 0.25) (layer "F.Cu") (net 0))
 (segment (start 93.98 111.08246) (end 95.07754 111.08246) (width 0.25) (layer "F.Cu") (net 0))
 (segment (start 99.06 111.08246) (end 99.06 110.76) (width 0.25) (layer "F.Cu") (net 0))
 (segment (start 97.23 99.838152) (end 105.41 91.658152) (width 0.25) (layer "F.Cu") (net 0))
 (segment (start 107.023103 101.6) (end 106.008309 100.585206) (width 0.25) (layer "F.Cu") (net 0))
 (segment (start 109.428878 54.188511) (end 107.95 55.667389) (width 0.25) (layer "F.Cu") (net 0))
 (segment (start 99.06 111.08246) (end 104.14 111.08246) (width 0.25) (layer "F.Cu") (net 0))
 (segment (start 124.46 111.08246) (end 125.55754 111.08246) (width 0.25) (layer "F.Cu") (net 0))
 (segment (start 119.38 110.76) (end 119.38 101.6) (width 0.25) (layer "F.Cu") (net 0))
 (segment (start 99.06 110.76) (end 100.89 108.93) (width 0.25) (layer "F.Cu") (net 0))
 (segment (start 100.89 104.43) (end 107.39 104.43) (width 0.25) (layer "F.Cu") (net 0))
 (segment (start 140.97 86.36) (end 143.51 88.9) (width 0.25) (layer "F.Cu") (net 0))
 (segment (start 131.37 104.43) (end 134.62 104.43) (width 0.25) (layer "F.Cu") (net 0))
 (segment (start 88.22246 111.08246) (end 88.57754 111.08246) (width 0.25) (layer "F.Cu") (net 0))
 (segment (start 129.54 111.08246) (end 129.54 110.76) (width 0.25) (layer "F.Cu") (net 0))
 (segment (start 88.9 99.06) (end 93.98 99.06) (width 0.25) (layer "F.Cu") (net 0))
 (segment (start 110.49 96.025811) (end 110.49 88.9) (width 0.25) (layer "F.Cu") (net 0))
 (segment (start 109.22 111.08246) (end 109.22 101.6) (width 0.25) (layer "F.Cu") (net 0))
 (segment (start 105.495659 57.513663) (end 105.136612 57.154616) (width 0.25) (layer "F.Cu") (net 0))
 (segment (start 134.62 104.43) (end 137.87 104.43) (width 0.25) (layer "F.Cu") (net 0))
 (segment (start 100.334616 57.154616) (end 99.06 55.88) (width 0.25) (layer "F.Cu") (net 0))
 (segment (start 106.677513 58.422487) (end 103.289539 58.422487) (width 0.25) (layer "B.Cu") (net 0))
 (segment (start 111.75 58.42) (end 111.75 62.008674) (width 0.25) (layer "B.Cu") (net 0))
 (segment (start 103.289539 58.422487) (end 101.597513 58.422487) (width 0.25) (layer "B.Cu") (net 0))
 (segment (start 103.077004 53.980352) (end 112.400352 53.980352) (width 0.25) (layer "B.Cu") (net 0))
 (segment (start 103.077004 53.980352) (end 103.289539 54.192887) (width 0.25) (layer "B.Cu") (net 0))
 (segment (start 111.75 58.42) (end 106.68 58.42) (width 0.25) (layer "B.Cu") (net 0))
 (segment (start 112.400352 53.980352) (end 114.29 55.87) (width 0.25) (layer "B.Cu") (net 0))
 (segment (start 106.68 58.42) (end 106.677513 58.422487) (width 0.25) (layer "B.Cu") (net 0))
 (segment (start 100.33 71.12) (end 100.33 66.462026) (width 0.25) (layer "B.Cu") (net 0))
 (segment (start 88.9 71.12) (end 91.44 71.12) (width 0.25) (layer "B.Cu") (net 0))
 (segment (start 101.597513 58.422487) (end 99.06 60.96) (width 0.25) (layer "B.Cu") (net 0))
 (segment (start 111.75 62.008674) (end 115.57 65.828674) (width 0.25) (layer "B.Cu") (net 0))
 (segment (start 93.98 68.58) (end 93.98 63.5) (width 0.25) (layer "B.Cu") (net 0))
 (segment (start 93.98 53.980352) (end 103.077004 53.980352) (width 0.25) (layer "B.Cu") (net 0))
 (segment (start 93.98 63.5) (end 93.98 53.980352) (width 0.25) (layer "B.Cu") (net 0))
 (segment (start 93.98 63.5) (end 99.06 63.5) (width 0.25) (layer "B.Cu") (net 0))
 (segment (start 100.33 66.462026) (end 103.289539 63.502487) (width 0.25) (layer "B.Cu") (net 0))
 (segment (start 103.289539 54.192887) (end 103.289539 55.882487) (width 0.25) (layer "B.Cu") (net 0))
 (segment (start 91.44 71.12) (end 93.98 68.58) (width 0.25) (layer "B.Cu") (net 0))
 (segment (start 114.29 55.87) (end 114.29 58.42) (width 0.25) (layer "B.Cu") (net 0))
 (segment (start 115.57 65.828674) (end 115.57 71.12) (width 0.25) (layer "B.Cu") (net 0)))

